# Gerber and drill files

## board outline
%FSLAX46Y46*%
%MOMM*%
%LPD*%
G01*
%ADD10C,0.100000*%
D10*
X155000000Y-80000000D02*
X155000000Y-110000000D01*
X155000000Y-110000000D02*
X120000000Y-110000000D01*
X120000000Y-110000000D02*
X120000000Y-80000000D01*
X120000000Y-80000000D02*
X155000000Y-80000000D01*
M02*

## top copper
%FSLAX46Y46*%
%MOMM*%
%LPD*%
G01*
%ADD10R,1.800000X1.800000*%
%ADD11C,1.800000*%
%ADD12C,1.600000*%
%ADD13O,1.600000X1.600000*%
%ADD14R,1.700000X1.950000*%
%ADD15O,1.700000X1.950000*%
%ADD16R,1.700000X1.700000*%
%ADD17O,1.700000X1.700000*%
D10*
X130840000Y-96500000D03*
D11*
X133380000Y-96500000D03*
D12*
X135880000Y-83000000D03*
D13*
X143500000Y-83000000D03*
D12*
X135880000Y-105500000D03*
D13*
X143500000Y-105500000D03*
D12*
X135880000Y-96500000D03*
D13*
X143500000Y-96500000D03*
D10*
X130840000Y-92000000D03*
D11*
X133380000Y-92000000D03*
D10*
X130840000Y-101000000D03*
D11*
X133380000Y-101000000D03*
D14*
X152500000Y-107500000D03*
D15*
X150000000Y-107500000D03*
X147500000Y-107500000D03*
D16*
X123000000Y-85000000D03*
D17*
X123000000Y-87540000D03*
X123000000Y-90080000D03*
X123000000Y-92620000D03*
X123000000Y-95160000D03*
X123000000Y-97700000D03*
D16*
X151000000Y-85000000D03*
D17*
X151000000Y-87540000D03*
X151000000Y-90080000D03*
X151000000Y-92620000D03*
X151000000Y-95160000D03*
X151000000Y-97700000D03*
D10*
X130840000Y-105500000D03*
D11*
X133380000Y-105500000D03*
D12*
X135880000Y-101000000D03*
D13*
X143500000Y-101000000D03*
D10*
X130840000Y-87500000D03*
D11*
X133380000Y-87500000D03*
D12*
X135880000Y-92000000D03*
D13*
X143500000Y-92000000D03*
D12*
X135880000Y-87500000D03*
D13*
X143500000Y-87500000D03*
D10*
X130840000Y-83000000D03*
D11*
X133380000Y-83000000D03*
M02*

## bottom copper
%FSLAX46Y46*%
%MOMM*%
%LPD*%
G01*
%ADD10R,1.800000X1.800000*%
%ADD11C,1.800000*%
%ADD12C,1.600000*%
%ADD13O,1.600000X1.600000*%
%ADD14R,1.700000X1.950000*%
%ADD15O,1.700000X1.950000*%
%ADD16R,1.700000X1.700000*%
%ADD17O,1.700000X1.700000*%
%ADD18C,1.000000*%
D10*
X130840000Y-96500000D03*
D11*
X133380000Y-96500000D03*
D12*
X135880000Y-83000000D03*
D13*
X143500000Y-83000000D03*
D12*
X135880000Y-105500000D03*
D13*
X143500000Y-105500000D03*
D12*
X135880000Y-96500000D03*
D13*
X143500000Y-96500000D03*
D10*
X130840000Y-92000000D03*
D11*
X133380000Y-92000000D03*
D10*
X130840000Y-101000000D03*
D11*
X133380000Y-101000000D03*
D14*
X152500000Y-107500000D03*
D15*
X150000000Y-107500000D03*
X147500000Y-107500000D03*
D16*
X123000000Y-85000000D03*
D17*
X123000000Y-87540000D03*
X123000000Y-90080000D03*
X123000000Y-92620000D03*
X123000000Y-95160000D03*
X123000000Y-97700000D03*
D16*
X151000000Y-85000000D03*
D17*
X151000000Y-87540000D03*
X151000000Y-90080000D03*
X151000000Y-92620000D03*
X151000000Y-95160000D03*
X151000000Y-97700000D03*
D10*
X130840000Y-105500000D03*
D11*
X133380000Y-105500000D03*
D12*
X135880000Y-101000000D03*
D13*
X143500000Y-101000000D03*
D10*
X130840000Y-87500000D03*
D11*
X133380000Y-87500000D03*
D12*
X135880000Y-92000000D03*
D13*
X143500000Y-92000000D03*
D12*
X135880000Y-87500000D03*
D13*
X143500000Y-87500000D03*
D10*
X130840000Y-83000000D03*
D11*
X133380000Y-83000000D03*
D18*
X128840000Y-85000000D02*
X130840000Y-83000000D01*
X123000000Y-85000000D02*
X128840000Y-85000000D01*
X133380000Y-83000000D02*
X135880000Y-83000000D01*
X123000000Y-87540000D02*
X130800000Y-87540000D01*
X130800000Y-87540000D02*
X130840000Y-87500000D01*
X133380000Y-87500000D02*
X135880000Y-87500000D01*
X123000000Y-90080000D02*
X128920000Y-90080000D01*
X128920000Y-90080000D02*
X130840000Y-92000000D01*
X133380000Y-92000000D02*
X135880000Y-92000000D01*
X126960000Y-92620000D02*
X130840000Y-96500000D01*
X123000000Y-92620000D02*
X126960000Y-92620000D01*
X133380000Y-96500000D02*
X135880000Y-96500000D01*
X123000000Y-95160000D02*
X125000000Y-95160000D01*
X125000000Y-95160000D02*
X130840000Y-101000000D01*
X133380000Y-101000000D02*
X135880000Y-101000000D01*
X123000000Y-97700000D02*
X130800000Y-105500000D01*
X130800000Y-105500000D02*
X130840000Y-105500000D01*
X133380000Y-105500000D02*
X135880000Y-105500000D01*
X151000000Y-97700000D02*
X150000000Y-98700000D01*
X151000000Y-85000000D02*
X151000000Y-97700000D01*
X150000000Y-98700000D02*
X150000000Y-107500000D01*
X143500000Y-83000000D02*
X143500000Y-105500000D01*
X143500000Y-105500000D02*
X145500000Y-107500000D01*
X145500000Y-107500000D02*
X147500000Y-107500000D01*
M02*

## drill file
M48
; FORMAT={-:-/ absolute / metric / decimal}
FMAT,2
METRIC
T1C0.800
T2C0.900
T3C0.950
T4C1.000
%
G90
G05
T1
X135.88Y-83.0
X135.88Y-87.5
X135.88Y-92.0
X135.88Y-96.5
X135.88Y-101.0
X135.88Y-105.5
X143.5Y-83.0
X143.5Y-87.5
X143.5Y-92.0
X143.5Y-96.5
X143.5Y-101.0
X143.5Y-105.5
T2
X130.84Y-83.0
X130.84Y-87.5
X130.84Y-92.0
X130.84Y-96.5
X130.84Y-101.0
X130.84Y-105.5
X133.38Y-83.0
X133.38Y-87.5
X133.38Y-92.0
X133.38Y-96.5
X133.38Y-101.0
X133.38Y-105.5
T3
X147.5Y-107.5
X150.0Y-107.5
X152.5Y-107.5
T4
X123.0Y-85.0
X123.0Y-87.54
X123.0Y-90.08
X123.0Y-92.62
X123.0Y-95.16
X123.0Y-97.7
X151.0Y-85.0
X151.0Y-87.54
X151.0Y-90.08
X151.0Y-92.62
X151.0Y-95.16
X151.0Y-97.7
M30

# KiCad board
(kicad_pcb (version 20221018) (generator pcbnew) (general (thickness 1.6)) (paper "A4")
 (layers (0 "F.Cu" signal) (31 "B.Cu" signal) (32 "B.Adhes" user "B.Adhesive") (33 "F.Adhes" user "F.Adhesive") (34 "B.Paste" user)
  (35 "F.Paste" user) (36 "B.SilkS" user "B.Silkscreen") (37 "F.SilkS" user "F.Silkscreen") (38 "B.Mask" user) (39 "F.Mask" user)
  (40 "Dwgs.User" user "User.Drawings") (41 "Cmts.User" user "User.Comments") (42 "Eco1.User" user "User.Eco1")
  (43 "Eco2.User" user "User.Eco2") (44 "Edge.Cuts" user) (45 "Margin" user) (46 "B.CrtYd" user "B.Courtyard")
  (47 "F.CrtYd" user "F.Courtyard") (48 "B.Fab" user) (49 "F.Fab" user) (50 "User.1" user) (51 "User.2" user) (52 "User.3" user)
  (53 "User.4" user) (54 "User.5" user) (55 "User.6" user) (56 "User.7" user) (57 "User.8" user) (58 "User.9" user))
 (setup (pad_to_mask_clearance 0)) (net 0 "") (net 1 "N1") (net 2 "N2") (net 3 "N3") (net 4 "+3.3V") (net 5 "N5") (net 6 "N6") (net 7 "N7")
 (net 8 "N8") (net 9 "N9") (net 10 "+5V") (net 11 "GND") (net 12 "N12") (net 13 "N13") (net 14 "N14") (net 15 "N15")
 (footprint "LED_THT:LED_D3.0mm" (layer "F.Cu") (at 130.84 96.5)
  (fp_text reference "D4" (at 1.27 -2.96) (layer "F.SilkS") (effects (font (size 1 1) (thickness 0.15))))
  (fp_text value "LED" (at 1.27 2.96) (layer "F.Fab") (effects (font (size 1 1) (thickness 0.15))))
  (pad "1" thru_hole rect (at 0 0) (size 1.8 1.8) (drill 0.9) (layers "*.Cu" "*.Mask") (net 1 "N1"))
  (pad "2" thru_hole circle (at 2.54 0) (size 1.8 1.8) (drill 0.9) (layers "*.Cu" "*.Mask") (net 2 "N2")))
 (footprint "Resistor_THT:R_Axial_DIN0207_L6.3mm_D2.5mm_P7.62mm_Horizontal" (layer "F.Cu") (at 135.88 83)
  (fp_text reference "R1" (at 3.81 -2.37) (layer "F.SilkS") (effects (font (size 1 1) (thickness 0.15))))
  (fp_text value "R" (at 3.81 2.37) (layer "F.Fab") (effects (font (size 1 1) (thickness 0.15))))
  (pad "1" thru_hole circle (at 0 0) (size 1.6 1.6) (drill 0.8) (layers "*.Cu" "*.Mask") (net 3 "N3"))
  (pad "2" thru_hole oval (at 7.62 0) (size 1.6 1.6) (drill 0.8) (layers "*.Cu" "*.Mask") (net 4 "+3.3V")))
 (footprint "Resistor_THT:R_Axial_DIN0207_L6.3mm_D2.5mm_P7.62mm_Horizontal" (layer "F.Cu") (at 135.88 105.5)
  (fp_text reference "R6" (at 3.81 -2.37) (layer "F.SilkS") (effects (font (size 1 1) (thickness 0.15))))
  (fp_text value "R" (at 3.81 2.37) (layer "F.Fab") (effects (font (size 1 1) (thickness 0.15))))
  (pad "1" thru_hole circle (at 0 0) (size 1.6 1.6) (drill 0.8) (layers "*.Cu" "*.Mask") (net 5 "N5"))
  (pad "2" thru_hole oval (at 7.62 0) (size 1.6 1.6) (drill 0.8) (layers "*.Cu" "*.Mask") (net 4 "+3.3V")))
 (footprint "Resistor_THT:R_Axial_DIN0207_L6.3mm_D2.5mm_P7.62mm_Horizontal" (layer "F.Cu") (at 135.88 96.5)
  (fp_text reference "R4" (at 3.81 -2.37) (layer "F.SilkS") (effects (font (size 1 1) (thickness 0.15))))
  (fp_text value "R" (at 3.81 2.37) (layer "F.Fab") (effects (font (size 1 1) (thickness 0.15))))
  (pad "1" thru_hole circle (at 0 0) (size 1.6 1.6) (drill 0.8) (layers "*.Cu" "*.Mask") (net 2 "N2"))
  (pad "2" thru_hole oval (at 7.62 0) (size 1.6 1.6) (drill 0.8) (layers "*.Cu" "*.Mask") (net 4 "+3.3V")))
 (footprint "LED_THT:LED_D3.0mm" (layer "F.Cu") (at 130.84 92)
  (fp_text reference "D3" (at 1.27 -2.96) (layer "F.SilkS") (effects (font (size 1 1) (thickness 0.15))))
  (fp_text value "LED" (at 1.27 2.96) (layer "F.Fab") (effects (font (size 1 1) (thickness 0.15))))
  (pad "1" thru_hole rect (at 0 0) (size 1.8 1.8) (drill 0.9) (layers "*.Cu" "*.Mask") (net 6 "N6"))
  (pad "2" thru_hole circle (at 2.54 0) (size 1.8 1.8) (drill 0.9) (layers "*.Cu" "*.Mask") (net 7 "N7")))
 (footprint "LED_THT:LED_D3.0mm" (layer "F.Cu") (at 130.84 101)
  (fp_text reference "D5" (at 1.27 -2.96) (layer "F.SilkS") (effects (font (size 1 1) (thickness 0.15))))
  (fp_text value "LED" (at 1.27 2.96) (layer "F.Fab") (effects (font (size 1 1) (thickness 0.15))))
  (pad "1" thru_hole rect (at 0 0) (size 1.8 1.8) (drill 0.9) (layers "*.Cu" "*.Mask") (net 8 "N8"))
  (pad "2" thru_hole circle (at 2.54 0) (size 1.8 1.8) (drill 0.9) (layers "*.Cu" "*.Mask") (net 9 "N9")))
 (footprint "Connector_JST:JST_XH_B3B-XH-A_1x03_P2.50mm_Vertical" (layer "F.Cu") (at 152.5 107.5 180)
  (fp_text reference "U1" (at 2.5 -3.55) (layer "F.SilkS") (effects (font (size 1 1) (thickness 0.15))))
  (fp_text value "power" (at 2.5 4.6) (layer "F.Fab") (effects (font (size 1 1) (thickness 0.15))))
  (pad "1" thru_hole rect (at 0 0 180) (size 1.7 1.95) (drill 0.95) (layers "*.Cu" "*.Mask") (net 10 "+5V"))
  (pad "2" thru_hole oval (at 2.5 0 180) (size 1.7 1.95) (drill 0.95) (layers "*.Cu" "*.Mask") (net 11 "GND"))
  (pad "3" thru_hole oval (at 5 0 180) (size 1.7 1.95) (drill 0.95) (layers "*.Cu" "*.Mask") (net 4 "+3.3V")))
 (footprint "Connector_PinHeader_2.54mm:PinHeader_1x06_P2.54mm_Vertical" (layer "F.Cu") (at 123 85)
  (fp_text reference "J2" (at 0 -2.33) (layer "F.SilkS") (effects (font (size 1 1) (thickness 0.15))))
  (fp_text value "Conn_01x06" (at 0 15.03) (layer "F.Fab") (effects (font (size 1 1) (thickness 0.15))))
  (pad "1" thru_hole rect (at 0 0) (size 1.7 1.7) (drill 1) (layers "*.Cu" "*.Mask") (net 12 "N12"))
  (pad "2" thru_hole oval (at 0 2.54) (size 1.7 1.7) (drill 1) (layers "*.Cu" "*.Mask") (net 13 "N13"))
  (pad "3" thru_hole oval (at 0 5.08) (size 1.7 1.7) (drill 1) (layers "*.Cu" "*.Mask") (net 6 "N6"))
  (pad "4" thru_hole oval (at 0 7.62) (size 1.7 1.7) (drill 1) (layers "*.Cu" "*.Mask") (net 1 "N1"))
  (pad "5" thru_hole oval (at 0 10.16) (size 1.7 1.7) (drill 1) (layers "*.Cu" "*.Mask") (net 8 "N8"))
  (pad "6" thru_hole oval (at 0 12.7) (size 1.7 1.7) (drill 1) (layers "*.Cu" "*.Mask") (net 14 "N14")))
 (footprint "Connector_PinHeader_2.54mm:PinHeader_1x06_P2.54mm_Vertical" (layer "F.Cu") (at 151 85)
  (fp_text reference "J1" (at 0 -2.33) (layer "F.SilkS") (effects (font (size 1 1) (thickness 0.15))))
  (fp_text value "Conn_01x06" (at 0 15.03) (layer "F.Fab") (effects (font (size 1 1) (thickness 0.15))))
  (pad "1" thru_hole rect (at 0 0) (size 1.7 1.7) (drill 1) (layers "*.Cu" "*.Mask") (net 11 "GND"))
  (pad "2" thru_hole oval (at 0 2.54) (size 1.7 1.7) (drill 1) (layers "*.Cu" "*.Mask") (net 11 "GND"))
  (pad "3" thru_hole oval (at 0 5.08) (size 1.7 1.7) (drill 1) (layers "*.Cu" "*.Mask") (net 11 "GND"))
  (pad "4" thru_hole oval (at 0 7.62) (size 1.7 1.7) (drill 1) (layers "*.Cu" "*.Mask") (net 11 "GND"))
  (pad "5" thru_hole oval (at 0 10.16) (size 1.7 1.7) (drill 1) (layers "*.Cu" "*.Mask") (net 11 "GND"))
  (pad "6" thru_hole oval (at 0 12.7) (size 1.7 1.7) (drill 1) (layers "*.Cu" "*.Mask") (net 11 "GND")))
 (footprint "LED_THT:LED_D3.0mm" (layer "F.Cu") (at 130.84 105.5)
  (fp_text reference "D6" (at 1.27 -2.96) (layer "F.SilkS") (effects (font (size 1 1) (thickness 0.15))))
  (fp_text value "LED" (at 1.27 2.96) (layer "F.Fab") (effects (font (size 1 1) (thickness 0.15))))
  (pad "1" thru_hole rect (at 0 0) (size 1.8 1.8) (drill 0.9) (layers "*.Cu" "*.Mask") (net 14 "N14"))
  (pad "2" thru_hole circle (at 2.54 0) (size 1.8 1.8) (drill 0.9) (layers "*.Cu" "*.Mask") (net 5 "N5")))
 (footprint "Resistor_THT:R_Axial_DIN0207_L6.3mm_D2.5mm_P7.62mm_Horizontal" (layer "F.Cu") (at 135.88 101)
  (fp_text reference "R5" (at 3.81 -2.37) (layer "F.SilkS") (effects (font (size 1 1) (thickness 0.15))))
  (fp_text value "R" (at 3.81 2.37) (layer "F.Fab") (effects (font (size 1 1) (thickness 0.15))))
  (pad "1" thru_hole circle (at 0 0) (size 1.6 1.6) (drill 0.8) (layers "*.Cu" "*.Mask") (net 9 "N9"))
  (pad "2" thru_hole oval (at 7.62 0) (size 1.6 1.6) (drill 0.8) (layers "*.Cu" "*.Mask") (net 4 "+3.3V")))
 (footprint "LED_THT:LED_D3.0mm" (layer "F.Cu") (at 130.84 87.5)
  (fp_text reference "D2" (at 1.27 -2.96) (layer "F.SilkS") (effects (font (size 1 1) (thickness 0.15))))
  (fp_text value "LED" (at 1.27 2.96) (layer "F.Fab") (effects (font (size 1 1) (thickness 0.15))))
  (pad "1" thru_hole rect (at 0 0) (size 1.8 1.8) (drill 0.9) (layers "*.Cu" "*.Mask") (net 13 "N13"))
  (pad "2" thru_hole circle (at 2.54 0) (size 1.8 1.8) (drill 0.9) (layers "*.Cu" "*.Mask") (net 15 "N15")))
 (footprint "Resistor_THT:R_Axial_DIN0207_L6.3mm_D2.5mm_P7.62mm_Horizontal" (layer "F.Cu") (at 135.88 92)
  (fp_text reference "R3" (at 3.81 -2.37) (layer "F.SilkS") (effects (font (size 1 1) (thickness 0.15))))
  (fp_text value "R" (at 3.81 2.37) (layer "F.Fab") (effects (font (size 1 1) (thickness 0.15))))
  (pad "1" thru_hole circle (at 0 0) (size 1.6 1.6) (drill 0.8) (layers "*.Cu" "*.Mask") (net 7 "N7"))
  (pad "2" thru_hole oval (at 7.62 0) (size 1.6 1.6) (drill 0.8) (layers "*.Cu" "*.Mask") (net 4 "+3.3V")))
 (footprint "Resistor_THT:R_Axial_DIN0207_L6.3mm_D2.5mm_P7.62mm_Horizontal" (layer "F.Cu") (at 135.88 87.5)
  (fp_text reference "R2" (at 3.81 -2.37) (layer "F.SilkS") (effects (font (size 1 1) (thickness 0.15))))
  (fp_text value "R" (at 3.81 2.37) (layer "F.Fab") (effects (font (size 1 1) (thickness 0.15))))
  (pad "1" thru_hole circle (at 0 0) (size 1.6 1.6) (drill 0.8) (layers "*.Cu" "*.Mask") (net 15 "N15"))
  (pad "2" thru_hole oval (at 7.62 0) (size 1.6 1.6) (drill 0.8) (layers "*.Cu" "*.Mask") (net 4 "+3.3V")))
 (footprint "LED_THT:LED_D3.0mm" (layer "F.Cu") (at 130.84 83)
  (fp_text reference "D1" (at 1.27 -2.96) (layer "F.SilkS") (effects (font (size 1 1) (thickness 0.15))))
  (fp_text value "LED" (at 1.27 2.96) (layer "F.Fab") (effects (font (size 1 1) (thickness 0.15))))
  (pad "1" thru_hole rect (at 0 0) (size 1.8 1.8) (drill 0.9) (layers "*.Cu" "*.Mask") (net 12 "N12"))
  (pad "2" thru_hole circle (at 2.54 0) (size 1.8 1.8) (drill 0.9) (layers "*.Cu" "*.Mask") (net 3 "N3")))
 (gr_line (start 155 80) (end 155 110) (stroke (width 0.1) (type default)) (layer "Edge.Cuts"))
 (gr_line (start 155 110) (end 120 110) (stroke (width 0.1) (type default)) (layer "Edge.Cuts"))
 (gr_line (start 120 110) (end 120 80) (stroke (width 0.1) (type default)) (layer "Edge.Cuts"))
 (gr_line (start 120 80) (end 155 80) (stroke (width 0.1) (type default)) (layer "Edge.Cuts"))
 (segment (start 128.84 85) (end 130.84 83) (width 1) (layer "B.Cu") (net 12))
 (segment (start 123 85) (end 128.84 85) (width 1) (layer "B.Cu") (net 12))
 (segment (start 133.38 83) (end 135.88 83) (width 1) (layer "B.Cu") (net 3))
 (segment (start 123 87.54) (end 130.8 87.54) (width 1) (layer "B.Cu") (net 13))
 (segment (start 130.8 87.54) (end 130.84 87.5) (width 1) (layer "B.Cu") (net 13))
 (segment (start 133.38 87.5) (end 135.88 87.5) (width 1) (layer "B.Cu") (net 15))
 (segment (start 123 90.08) (end 128.92 90.08) (width 1) (layer "B.Cu") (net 6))
 (segment (start 128.92 90.08) (end 130.84 92) (width 1) (layer "B.Cu") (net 6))
 (segment (start 133.38 92) (end 135.88 92) (width 1) (layer "B.Cu") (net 7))
 (segment (start 126.96 92.62) (end 130.84 96.5) (width 1) (layer "B.Cu") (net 1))
 (segment (start 123 92.62) (end 126.96 92.62) (width 1) (layer "B.Cu") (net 1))
 (segment (start 133.38 96.5) (end 135.88 96.5) (width 1) (layer "B.Cu") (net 2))
 (segment (start 123 95.16) (end 125 95.16) (width 1) (layer "B.Cu") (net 8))
 (segment (start 125 95.16) (end 130.84 101) (width 1) (layer "B.Cu") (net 8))
 (segment (start 133.38 101) (end 135.88 101) (width 1) (layer "B.Cu") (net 9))
 (segment (start 123 97.7) (end 130.8 105.5) (width 1) (layer "B.Cu") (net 14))
 (segment (start 130.8 105.5) (end 130.84 105.5) (width 1) (layer "B.Cu") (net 14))
 (segment (start 133.38 105.5) (end 135.88 105.5) (width 1) (layer "B.Cu") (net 5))
 (segment (start 151 97.7) (end 150 98.7) (width 1) (layer "B.Cu") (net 11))
 (segment (start 151 85) (end 151 97.7) (width 1) (layer "B.Cu") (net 11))
 (segment (start 150 98.7) (end 150 107.5) (width 1) (layer "B.Cu") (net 11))
 (segment (start 143.5 83) (end 143.5 105.5) (width 1) (layer "B.Cu") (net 4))
 (segment (start 143.5 105.5) (end 145.5 107.5) (width 1) (layer "B.Cu") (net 4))
 (segment (start 145.5 107.5) (end 147.5 107.5) (width 1) (layer "B.Cu") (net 4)))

